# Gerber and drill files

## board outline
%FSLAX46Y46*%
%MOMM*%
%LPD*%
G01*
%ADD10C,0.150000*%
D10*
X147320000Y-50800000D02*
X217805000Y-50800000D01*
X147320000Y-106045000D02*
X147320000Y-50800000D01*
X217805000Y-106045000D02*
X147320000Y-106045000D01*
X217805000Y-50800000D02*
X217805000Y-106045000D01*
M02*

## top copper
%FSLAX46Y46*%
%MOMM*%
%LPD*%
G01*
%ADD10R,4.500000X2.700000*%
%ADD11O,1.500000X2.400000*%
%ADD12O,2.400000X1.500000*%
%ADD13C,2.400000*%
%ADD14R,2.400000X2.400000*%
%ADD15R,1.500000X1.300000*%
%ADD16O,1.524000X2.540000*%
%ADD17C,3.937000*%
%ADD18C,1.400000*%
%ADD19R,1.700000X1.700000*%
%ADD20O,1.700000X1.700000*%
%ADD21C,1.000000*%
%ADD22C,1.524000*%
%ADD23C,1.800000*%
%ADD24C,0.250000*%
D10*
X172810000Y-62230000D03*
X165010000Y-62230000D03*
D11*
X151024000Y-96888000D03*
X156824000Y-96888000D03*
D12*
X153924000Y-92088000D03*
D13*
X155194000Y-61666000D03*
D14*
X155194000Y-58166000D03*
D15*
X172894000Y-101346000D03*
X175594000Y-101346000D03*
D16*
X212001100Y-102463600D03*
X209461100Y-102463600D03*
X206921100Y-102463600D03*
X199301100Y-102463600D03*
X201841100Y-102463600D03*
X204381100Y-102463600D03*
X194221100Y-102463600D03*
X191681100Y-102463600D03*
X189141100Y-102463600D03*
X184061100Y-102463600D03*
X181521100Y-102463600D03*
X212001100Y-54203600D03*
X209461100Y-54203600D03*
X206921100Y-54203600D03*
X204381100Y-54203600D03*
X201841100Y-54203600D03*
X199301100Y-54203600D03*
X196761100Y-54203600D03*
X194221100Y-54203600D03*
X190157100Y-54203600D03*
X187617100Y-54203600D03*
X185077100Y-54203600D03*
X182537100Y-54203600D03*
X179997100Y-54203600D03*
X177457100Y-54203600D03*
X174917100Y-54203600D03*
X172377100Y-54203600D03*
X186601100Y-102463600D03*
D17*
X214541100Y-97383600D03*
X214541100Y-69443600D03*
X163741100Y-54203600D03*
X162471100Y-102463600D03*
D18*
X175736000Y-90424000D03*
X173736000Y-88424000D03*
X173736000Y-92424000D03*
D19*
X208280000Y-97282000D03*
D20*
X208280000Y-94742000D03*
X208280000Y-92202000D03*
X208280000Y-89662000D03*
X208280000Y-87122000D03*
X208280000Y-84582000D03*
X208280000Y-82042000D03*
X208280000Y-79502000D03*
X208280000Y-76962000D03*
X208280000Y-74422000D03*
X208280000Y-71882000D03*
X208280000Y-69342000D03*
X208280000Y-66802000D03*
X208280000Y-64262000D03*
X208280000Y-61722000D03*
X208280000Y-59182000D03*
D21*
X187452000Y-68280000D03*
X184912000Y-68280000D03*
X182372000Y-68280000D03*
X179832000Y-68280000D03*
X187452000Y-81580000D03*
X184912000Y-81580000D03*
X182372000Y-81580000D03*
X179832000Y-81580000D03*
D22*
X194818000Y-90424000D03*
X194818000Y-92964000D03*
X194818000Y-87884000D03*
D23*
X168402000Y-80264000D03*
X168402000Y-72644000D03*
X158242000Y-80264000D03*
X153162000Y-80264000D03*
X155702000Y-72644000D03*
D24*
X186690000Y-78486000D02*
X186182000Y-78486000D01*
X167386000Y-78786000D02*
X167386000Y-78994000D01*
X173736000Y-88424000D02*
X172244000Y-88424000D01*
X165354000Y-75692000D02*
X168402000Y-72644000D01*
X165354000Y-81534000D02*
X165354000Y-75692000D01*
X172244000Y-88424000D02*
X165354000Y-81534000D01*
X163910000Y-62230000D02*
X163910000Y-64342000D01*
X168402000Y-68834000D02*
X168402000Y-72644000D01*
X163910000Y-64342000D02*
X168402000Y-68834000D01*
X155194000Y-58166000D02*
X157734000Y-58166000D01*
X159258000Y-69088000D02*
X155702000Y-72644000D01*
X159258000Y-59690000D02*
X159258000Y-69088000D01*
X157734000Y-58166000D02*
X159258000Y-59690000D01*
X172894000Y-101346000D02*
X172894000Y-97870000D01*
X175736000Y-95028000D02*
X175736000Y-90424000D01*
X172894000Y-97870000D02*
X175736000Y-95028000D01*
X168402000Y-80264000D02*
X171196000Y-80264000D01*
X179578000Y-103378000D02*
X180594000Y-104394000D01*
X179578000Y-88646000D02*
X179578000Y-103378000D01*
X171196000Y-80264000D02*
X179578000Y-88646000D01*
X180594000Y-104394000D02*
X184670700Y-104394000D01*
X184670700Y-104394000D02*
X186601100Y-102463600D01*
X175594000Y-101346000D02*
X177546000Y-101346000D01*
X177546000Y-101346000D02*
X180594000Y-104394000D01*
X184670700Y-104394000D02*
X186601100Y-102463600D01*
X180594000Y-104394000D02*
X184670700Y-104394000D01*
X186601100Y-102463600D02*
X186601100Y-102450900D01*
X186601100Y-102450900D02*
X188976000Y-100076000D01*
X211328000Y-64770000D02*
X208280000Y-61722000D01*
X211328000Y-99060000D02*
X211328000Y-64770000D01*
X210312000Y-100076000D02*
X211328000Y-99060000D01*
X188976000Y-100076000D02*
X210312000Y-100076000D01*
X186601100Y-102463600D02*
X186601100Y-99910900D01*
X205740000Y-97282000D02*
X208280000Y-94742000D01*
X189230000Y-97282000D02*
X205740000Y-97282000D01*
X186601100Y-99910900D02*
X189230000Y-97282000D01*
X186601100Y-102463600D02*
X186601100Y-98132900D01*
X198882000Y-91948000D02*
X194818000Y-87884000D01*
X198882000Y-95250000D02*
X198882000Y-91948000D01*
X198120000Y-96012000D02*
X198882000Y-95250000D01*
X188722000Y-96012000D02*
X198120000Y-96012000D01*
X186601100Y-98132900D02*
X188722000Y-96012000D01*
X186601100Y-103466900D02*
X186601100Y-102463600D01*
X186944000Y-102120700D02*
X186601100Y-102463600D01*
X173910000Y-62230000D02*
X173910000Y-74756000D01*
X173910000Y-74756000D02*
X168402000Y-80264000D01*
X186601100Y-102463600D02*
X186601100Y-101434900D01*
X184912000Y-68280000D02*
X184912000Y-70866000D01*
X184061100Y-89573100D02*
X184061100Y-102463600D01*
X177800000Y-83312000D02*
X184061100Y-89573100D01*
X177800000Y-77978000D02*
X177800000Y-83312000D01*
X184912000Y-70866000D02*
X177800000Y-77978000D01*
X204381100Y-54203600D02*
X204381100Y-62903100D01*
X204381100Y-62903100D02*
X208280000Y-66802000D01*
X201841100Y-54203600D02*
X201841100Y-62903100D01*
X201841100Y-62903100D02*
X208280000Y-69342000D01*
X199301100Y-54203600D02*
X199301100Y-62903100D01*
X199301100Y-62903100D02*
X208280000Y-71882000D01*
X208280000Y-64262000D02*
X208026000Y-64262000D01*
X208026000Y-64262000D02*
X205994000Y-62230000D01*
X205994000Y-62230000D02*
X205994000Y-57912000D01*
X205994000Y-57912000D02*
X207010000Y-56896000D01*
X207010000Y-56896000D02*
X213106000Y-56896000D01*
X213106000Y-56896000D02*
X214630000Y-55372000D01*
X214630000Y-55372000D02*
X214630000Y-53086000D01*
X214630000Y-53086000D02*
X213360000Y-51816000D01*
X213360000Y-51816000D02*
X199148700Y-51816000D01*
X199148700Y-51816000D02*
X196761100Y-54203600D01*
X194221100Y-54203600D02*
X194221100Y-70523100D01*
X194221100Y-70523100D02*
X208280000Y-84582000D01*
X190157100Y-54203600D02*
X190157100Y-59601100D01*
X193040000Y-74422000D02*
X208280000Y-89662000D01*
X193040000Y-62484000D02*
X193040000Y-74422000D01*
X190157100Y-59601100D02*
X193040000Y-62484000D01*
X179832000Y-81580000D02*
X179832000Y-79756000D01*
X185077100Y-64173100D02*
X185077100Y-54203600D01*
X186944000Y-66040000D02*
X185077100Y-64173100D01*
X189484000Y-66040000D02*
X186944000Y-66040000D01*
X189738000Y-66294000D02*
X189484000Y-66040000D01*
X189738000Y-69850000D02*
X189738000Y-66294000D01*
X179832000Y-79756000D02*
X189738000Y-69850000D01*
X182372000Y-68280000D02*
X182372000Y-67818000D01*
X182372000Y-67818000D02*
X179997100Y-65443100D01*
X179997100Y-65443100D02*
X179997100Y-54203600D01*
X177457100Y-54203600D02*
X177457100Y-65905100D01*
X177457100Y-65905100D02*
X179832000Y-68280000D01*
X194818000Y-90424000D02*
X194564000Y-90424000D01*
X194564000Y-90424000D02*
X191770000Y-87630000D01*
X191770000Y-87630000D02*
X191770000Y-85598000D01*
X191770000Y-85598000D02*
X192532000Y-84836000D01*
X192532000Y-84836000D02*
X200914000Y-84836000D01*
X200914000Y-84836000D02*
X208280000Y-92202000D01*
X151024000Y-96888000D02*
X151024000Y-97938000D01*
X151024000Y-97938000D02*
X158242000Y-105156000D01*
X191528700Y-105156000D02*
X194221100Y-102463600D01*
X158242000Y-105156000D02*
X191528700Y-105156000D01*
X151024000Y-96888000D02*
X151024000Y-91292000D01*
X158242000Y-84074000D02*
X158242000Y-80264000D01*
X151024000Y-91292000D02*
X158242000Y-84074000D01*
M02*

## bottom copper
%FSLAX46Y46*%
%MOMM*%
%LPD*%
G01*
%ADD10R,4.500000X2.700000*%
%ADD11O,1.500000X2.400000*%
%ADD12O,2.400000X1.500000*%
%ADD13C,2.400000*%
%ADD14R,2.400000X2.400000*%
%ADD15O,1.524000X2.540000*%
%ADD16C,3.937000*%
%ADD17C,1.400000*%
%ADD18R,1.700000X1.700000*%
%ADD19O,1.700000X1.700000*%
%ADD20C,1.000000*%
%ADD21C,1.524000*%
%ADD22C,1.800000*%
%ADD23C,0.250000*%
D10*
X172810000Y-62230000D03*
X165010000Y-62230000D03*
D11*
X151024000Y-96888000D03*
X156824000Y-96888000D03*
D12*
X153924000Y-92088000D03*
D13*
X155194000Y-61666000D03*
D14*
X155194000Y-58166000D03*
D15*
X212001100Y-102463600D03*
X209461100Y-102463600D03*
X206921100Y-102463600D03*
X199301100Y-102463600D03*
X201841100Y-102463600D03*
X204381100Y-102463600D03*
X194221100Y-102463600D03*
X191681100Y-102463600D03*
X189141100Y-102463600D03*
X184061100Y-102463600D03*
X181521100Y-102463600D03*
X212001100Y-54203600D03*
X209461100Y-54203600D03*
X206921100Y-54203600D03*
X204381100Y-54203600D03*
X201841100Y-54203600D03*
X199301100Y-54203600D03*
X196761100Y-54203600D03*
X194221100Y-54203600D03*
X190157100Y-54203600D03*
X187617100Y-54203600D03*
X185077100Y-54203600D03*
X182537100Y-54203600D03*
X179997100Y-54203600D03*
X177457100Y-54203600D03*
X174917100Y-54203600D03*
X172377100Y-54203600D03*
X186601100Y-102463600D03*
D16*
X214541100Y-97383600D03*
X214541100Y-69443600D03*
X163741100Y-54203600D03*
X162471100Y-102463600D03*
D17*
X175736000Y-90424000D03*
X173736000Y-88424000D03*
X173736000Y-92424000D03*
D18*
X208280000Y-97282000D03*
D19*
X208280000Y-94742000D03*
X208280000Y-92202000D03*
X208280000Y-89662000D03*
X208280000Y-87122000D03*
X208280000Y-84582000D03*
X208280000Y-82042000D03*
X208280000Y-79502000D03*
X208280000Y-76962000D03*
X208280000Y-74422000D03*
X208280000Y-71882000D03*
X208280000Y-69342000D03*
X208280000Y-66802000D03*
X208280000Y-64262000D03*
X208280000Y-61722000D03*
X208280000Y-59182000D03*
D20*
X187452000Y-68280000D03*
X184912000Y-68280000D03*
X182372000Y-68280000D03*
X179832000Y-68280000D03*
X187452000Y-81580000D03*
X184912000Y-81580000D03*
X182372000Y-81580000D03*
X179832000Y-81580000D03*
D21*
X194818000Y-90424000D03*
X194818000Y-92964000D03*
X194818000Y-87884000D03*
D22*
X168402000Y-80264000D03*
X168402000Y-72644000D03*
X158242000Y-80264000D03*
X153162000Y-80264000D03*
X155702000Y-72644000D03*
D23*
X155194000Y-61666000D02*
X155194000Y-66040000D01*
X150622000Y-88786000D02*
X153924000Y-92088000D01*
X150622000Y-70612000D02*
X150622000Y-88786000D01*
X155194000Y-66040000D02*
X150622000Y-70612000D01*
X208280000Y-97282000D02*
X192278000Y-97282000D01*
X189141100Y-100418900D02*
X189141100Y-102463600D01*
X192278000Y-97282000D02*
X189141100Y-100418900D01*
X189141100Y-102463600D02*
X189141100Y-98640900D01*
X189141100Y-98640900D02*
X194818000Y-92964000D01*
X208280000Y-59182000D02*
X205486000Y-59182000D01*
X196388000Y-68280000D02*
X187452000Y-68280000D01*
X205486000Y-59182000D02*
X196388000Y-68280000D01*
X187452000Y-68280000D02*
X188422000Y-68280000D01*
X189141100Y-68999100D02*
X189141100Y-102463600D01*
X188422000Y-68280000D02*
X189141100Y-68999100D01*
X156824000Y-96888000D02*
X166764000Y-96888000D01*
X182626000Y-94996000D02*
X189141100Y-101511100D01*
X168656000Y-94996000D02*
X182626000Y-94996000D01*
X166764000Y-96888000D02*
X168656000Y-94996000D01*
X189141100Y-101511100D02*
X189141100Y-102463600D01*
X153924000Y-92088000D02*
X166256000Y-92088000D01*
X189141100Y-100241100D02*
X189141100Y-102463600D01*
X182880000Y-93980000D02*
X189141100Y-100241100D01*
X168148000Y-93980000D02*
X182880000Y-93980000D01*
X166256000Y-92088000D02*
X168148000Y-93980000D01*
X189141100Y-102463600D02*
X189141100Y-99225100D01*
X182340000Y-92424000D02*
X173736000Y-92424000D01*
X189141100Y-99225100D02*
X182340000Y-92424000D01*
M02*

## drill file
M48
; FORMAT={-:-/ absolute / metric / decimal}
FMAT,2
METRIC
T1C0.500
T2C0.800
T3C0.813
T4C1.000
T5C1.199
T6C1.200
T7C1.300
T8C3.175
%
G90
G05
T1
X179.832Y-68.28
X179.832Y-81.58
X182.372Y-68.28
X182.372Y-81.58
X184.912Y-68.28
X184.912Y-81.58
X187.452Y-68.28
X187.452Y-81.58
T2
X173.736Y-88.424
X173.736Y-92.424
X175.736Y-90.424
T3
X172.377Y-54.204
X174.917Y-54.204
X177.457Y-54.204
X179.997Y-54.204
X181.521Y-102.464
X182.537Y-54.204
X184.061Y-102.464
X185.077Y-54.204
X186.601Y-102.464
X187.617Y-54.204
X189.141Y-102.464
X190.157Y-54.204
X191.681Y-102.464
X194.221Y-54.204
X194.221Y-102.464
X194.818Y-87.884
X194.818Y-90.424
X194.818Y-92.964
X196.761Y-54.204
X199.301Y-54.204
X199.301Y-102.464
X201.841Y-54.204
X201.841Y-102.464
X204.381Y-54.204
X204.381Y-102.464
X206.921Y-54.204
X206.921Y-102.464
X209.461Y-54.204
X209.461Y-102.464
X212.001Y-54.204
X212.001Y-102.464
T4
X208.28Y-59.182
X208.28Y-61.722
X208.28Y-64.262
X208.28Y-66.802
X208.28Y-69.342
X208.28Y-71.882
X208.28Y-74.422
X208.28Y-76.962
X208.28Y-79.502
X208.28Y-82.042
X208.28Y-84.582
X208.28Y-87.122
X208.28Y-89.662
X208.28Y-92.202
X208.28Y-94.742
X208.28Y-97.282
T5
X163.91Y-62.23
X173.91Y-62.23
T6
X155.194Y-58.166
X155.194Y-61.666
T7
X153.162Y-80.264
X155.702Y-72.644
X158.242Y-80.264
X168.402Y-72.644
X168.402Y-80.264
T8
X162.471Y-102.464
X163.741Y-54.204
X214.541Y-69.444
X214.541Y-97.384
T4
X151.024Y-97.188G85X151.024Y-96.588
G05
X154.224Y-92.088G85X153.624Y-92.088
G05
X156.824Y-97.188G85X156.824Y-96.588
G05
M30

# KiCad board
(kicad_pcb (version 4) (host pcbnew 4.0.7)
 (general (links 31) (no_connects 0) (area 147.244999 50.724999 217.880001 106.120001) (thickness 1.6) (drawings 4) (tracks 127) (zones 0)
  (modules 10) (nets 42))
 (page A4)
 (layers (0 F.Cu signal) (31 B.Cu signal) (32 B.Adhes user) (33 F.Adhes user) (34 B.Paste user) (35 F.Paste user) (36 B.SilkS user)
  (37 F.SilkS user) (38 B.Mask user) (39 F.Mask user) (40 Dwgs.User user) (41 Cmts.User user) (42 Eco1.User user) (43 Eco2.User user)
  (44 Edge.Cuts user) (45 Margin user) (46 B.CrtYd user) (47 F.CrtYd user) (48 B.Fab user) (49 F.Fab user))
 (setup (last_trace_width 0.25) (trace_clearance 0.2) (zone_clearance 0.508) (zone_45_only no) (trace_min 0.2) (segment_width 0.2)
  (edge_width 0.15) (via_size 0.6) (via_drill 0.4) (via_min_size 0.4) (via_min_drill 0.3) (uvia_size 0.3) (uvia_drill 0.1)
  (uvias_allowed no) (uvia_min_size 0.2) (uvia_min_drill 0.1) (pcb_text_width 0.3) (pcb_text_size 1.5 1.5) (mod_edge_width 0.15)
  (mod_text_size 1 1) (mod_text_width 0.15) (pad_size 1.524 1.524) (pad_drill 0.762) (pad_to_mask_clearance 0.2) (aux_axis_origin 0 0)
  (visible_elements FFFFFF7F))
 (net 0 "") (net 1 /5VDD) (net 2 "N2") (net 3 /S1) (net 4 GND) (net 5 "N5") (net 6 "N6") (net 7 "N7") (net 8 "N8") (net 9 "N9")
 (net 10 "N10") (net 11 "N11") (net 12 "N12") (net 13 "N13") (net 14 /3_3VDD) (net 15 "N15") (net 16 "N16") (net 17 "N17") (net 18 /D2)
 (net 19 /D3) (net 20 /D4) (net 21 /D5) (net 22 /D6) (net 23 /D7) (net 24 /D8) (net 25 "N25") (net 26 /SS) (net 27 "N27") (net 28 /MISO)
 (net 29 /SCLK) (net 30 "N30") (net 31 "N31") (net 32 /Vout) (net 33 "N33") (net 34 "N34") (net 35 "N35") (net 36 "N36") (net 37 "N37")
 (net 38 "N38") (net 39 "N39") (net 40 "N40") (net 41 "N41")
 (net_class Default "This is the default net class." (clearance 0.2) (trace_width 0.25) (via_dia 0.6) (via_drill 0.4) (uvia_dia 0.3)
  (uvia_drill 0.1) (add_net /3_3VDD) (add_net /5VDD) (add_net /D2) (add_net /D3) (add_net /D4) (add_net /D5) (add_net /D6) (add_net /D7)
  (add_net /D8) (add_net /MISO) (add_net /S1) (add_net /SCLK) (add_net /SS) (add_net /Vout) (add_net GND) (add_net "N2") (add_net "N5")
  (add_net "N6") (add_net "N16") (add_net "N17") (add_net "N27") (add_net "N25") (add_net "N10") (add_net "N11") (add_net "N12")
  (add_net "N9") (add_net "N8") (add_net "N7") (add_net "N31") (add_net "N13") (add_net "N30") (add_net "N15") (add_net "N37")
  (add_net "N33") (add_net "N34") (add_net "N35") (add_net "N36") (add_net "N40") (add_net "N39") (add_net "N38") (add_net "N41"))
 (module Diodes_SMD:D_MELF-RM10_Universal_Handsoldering (layer F.Cu) (at 168.91 62.23 180)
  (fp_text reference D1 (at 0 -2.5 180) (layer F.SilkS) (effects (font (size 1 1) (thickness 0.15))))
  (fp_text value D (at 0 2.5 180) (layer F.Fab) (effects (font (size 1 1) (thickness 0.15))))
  (pad 1 thru_hole rect (at -5 0 180) (size 4.5 2.7) (drill 1.19888 (offset 1.1 0)) (layers *.Cu *.Mask) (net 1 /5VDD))
  (pad 2 thru_hole rect (at 5 0) (size 4.5 2.7) (drill 1.19888 (offset 1.1 0)) (layers *.Cu *.Mask) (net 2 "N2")))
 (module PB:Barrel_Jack (layer F.Cu) (at 153.924 94.488 180)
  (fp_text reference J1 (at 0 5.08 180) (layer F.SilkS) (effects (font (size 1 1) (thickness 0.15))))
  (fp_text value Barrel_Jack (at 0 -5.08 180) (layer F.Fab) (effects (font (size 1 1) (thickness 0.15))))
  (pad 1 thru_hole oval (at 2.9 -2.4 180) (size 1.5 2.4) (drill oval 1 1.6) (layers *.Cu *.Mask) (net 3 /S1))
  (pad 2 thru_hole oval (at -2.9 -2.4 180) (size 1.5 2.4) (drill oval 1 1.6) (layers *.Cu *.Mask) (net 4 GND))
  (pad 3 thru_hole oval (at 0 2.4 180) (size 2.4 1.5) (drill oval 1.6 1) (layers *.Cu *.Mask) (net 4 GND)))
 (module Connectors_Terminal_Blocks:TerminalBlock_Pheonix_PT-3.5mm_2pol (layer F.Cu) (at 155.194 58.166 270)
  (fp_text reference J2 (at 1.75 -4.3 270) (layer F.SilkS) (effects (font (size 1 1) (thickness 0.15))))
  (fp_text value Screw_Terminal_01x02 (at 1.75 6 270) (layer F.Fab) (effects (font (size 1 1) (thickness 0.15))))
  (pad 2 thru_hole circle (at 3.5 0 270) (size 2.4 2.4) (drill 1.2) (layers *.Cu *.Mask) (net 4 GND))
  (pad 1 thru_hole rect (at 0 0 270) (size 2.4 2.4) (drill 1.2) (layers *.Cu *.Mask) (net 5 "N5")))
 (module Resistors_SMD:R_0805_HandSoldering (layer F.Cu) (at 174.244 101.346)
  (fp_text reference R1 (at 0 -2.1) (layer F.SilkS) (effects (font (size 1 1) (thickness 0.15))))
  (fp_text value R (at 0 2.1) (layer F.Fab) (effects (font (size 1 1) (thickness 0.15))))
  (pad 1 smd rect (at -1.35 0) (size 1.5 1.3) (layers F.Cu F.Paste F.Mask) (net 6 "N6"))
  (pad 2 smd rect (at 1.35 0) (size 1.5 1.3) (layers F.Cu F.Paste F.Mask) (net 1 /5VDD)))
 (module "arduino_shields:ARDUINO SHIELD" (layer F.Cu) (at 148.5011 105.0036)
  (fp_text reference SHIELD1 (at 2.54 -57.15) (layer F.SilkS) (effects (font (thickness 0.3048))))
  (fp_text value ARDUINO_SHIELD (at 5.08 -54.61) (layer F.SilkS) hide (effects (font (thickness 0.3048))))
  (pad AD5 thru_hole oval (at 63.5 -2.54 90) (size 2.54 1.524) (drill 0.8128) (layers *.Cu *.Mask F.SilkS) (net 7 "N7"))
  (pad AD4 thru_hole oval (at 60.96 -2.54 90) (size 2.54 1.524) (drill 0.8128) (layers *.Cu *.Mask F.SilkS) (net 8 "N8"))
  (pad AD3 thru_hole oval (at 58.42 -2.54 90) (size 2.54 1.524) (drill 0.8128) (layers *.Cu *.Mask F.SilkS) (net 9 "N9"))
  (pad AD0 thru_hole oval (at 50.8 -2.54 90) (size 2.54 1.524) (drill 0.8128) (layers *.Cu *.Mask F.SilkS) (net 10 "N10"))
  (pad AD1 thru_hole oval (at 53.34 -2.54 90) (size 2.54 1.524) (drill 0.8128) (layers *.Cu *.Mask F.SilkS) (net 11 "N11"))
  (pad AD2 thru_hole oval (at 55.88 -2.54 90) (size 2.54 1.524) (drill 0.8128) (layers *.Cu *.Mask F.SilkS) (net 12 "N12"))
  (pad V_IN thru_hole oval (at 45.72 -2.54 90) (size 2.54 1.524) (drill 0.8128) (layers *.Cu *.Mask F.SilkS) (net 3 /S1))
  (pad GND2 thru_hole oval (at 43.18 -2.54 90) (size 2.54 1.524) (drill 0.8128) (layers *.Cu *.Mask F.SilkS) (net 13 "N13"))
  (pad GND1 thru_hole oval (at 40.64 -2.54 90) (size 2.54 1.524) (drill 0.8128) (layers *.Cu *.Mask F.SilkS) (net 4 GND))
  (pad 3V3 thru_hole oval (at 35.56 -2.54 90) (size 2.54 1.524) (drill 0.8128) (layers *.Cu *.Mask F.SilkS) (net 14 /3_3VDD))
  (pad RST thru_hole oval (at 33.02 -2.54 90) (size 2.54 1.524) (drill 0.8128) (layers *.Cu *.Mask F.SilkS) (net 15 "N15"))
  (pad 0 thru_hole oval (at 63.5 -50.8 90) (size 2.54 1.524) (drill 0.8128) (layers *.Cu *.Mask F.SilkS) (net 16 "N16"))
  (pad 1 thru_hole oval (at 60.96 -50.8 90) (size 2.54 1.524) (drill 0.8128) (layers *.Cu *.Mask F.SilkS) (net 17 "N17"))
  (pad 2 thru_hole oval (at 58.42 -50.8 90) (size 2.54 1.524) (drill 0.8128) (layers *.Cu *.Mask F.SilkS) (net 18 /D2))
  (pad 3 thru_hole oval (at 55.88 -50.8 90) (size 2.54 1.524) (drill 0.8128) (layers *.Cu *.Mask F.SilkS) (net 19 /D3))
  (pad 4 thru_hole oval (at 53.34 -50.8 90) (size 2.54 1.524) (drill 0.8128) (layers *.Cu *.Mask F.SilkS) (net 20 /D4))
  (pad 5 thru_hole oval (at 50.8 -50.8 90) (size 2.54 1.524) (drill 0.8128) (layers *.Cu *.Mask F.SilkS) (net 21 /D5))
  (pad 6 thru_hole oval (at 48.26 -50.8 90) (size 2.54 1.524) (drill 0.8128) (layers *.Cu *.Mask F.SilkS) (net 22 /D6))
  (pad 7 thru_hole oval (at 45.72 -50.8 90) (size 2.54 1.524) (drill 0.8128) (layers *.Cu *.Mask F.SilkS) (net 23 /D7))
  (pad 8 thru_hole oval (at 41.656 -50.8 90) (size 2.54 1.524) (drill 0.8128) (layers *.Cu *.Mask F.SilkS) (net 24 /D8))
  (pad 9 thru_hole oval (at 39.116 -50.8 90) (size 2.54 1.524) (drill 0.8128) (layers *.Cu *.Mask F.SilkS) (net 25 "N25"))
  (pad 10 thru_hole oval (at 36.576 -50.8 90) (size 2.54 1.524) (drill 0.8128) (layers *.Cu *.Mask F.SilkS) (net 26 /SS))
  (pad 11 thru_hole oval (at 34.036 -50.8 90) (size 2.54 1.524) (drill 0.8128) (layers *.Cu *.Mask F.SilkS) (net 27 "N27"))
  (pad 12 thru_hole oval (at 31.496 -50.8 90) (size 2.54 1.524) (drill 0.8128) (layers *.Cu *.Mask F.SilkS) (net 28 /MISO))
  (pad 13 thru_hole oval (at 28.956 -50.8 90) (size 2.54 1.524) (drill 0.8128) (layers *.Cu *.Mask F.SilkS) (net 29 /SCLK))
  (pad GND3 thru_hole oval (at 26.416 -50.8 90) (size 2.54 1.524) (drill 0.8128) (layers *.Cu *.Mask F.SilkS) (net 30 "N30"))
  (pad AREF thru_hole oval (at 23.876 -50.8 90) (size 2.54 1.524) (drill 0.8128) (layers *.Cu *.Mask F.SilkS) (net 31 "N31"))
  (pad 5V thru_hole oval (at 38.1 -2.54 90) (size 2.54 1.524) (drill 0.8128) (layers *.Cu *.Mask F.SilkS) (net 1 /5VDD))
  (pad "" thru_hole circle (at 66.04 -7.62 90) (size 3.937 3.937) (drill 3.175) (layers *.Cu *.Mask F.SilkS))
  (pad "" thru_hole circle (at 66.04 -35.56 90) (size 3.937 3.937) (drill 3.175) (layers *.Cu *.Mask F.SilkS))
  (pad "" thru_hole circle (at 15.24 -50.8 90) (size 3.937 3.937) (drill 3.175) (layers *.Cu *.Mask F.SilkS))
  (pad "" thru_hole circle (at 13.97 -2.54 90) (size 3.937 3.937) (drill 3.175) (layers *.Cu *.Mask F.SilkS)))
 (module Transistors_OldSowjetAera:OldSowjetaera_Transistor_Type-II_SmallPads (layer F.Cu) (at 173.736 90.424 270)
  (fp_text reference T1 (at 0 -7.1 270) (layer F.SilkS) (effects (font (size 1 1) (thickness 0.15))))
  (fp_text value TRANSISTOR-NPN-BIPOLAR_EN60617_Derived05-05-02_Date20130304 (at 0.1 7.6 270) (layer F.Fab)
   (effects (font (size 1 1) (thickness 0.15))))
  (pad 2 thru_hole circle (at 0 -2 270) (size 1.4 1.4) (drill 0.8) (layers *.Cu *.Mask) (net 6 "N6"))
  (pad 1 thru_hole circle (at -2 0 270) (size 1.4 1.4) (drill 0.8) (layers *.Cu *.Mask) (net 2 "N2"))
  (pad 3 thru_hole circle (at 2 0 270) (size 1.4 1.4) (drill 0.8) (layers *.Cu *.Mask) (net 4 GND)))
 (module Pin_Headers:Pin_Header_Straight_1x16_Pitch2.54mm (layer F.Cu) (at 208.28 97.282 180)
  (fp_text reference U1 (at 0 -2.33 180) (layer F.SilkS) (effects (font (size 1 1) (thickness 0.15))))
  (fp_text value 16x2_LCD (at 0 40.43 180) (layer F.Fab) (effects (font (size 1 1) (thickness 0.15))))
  (pad 1 thru_hole rect (at 0 0 180) (size 1.7 1.7) (drill 1) (layers *.Cu *.Mask) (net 4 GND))
  (pad 2 thru_hole oval (at 0 2.54 180) (size 1.7 1.7) (drill 1) (layers *.Cu *.Mask) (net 1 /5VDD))
  (pad 3 thru_hole oval (at 0 5.08 180) (size 1.7 1.7) (drill 1) (layers *.Cu *.Mask) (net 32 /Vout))
  (pad 4 thru_hole oval (at 0 7.62 180) (size 1.7 1.7) (drill 1) (layers *.Cu *.Mask) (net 24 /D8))
  (pad 5 thru_hole oval (at 0 10.16 180) (size 1.7 1.7) (drill 1) (layers *.Cu *.Mask) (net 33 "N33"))
  (pad 6 thru_hole oval (at 0 12.7 180) (size 1.7 1.7) (drill 1) (layers *.Cu *.Mask) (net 23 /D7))
  (pad 7 thru_hole oval (at 0 15.24 180) (size 1.7 1.7) (drill 1) (layers *.Cu *.Mask) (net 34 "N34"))
  (pad 8 thru_hole oval (at 0 17.78 180) (size 1.7 1.7) (drill 1) (layers *.Cu *.Mask) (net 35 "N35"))
  (pad 9 thru_hole oval (at 0 20.32 180) (size 1.7 1.7) (drill 1) (layers *.Cu *.Mask) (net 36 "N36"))
  (pad 10 thru_hole oval (at 0 22.86 180) (size 1.7 1.7) (drill 1) (layers *.Cu *.Mask) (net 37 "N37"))
  (pad 11 thru_hole oval (at 0 25.4 180) (size 1.7 1.7) (drill 1) (layers *.Cu *.Mask) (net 21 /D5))
  (pad 12 thru_hole oval (at 0 27.94 180) (size 1.7 1.7) (drill 1) (layers *.Cu *.Mask) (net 20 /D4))
  (pad 13 thru_hole oval (at 0 30.48 180) (size 1.7 1.7) (drill 1) (layers *.Cu *.Mask) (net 19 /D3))
  (pad 14 thru_hole oval (at 0 33.02 180) (size 1.7 1.7) (drill 1) (layers *.Cu *.Mask) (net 22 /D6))
  (pad 15 thru_hole oval (at 0 35.56 180) (size 1.7 1.7) (drill 1) (layers *.Cu *.Mask) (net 1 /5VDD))
  (pad 16 thru_hole oval (at 0 38.1 180) (size 1.7 1.7) (drill 1) (layers *.Cu *.Mask) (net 4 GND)))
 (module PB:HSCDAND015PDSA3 (layer F.Cu) (at 183.642 74.93 270)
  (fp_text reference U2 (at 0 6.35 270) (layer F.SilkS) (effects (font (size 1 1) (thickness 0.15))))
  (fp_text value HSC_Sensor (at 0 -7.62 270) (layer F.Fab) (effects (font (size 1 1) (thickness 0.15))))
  (pad 1 thru_hole circle (at -6.65 -3.81 270) (size 1 1) (drill 0.5) (layers *.Cu *.Mask) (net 4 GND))
  (pad 2 thru_hole circle (at -6.65 -1.27 270) (size 1 1) (drill 0.5) (layers *.Cu *.Mask) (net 14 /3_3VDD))
  (pad 3 thru_hole circle (at -6.65 1.27 270) (size 1 1) (drill 0.5) (layers *.Cu *.Mask) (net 28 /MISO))
  (pad 4 thru_hole circle (at -6.65 3.81 270) (size 1 1) (drill 0.5) (layers *.Cu *.Mask) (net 29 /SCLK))
  (pad 8 thru_hole circle (at 6.65 -3.81 270) (size 1 1) (drill 0.5) (layers *.Cu *.Mask) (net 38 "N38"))
  (pad 7 thru_hole circle (at 6.65 -1.27 270) (size 1 1) (drill 0.5) (layers *.Cu *.Mask) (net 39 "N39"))
  (pad 6 thru_hole circle (at 6.65 1.27 270) (size 1 1) (drill 0.5) (layers *.Cu *.Mask) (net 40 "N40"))
  (pad 5 thru_hole circle (at 6.65 3.81 270) (size 1 1) (drill 0.5) (layers *.Cu *.Mask) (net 26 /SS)))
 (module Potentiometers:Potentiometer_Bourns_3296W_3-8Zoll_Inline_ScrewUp (layer F.Cu) (at 194.818 87.884 180)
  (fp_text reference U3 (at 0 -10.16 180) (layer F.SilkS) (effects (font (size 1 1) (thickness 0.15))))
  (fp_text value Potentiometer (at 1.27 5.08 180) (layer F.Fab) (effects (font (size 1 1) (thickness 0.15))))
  (pad 2 thru_hole circle (at 0 -2.54 180) (size 1.524 1.524) (drill 0.8128) (layers *.Cu *.Mask) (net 32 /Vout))
  (pad 3 thru_hole circle (at 0 -5.08 180) (size 1.524 1.524) (drill 0.8128) (layers *.Cu *.Mask) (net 4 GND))
  (pad 1 thru_hole circle (at 0 0 180) (size 1.524 1.524) (drill 0.8128) (layers *.Cu *.Mask) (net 1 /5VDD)))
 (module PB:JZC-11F (layer F.Cu) (at 162.052 76.454 90)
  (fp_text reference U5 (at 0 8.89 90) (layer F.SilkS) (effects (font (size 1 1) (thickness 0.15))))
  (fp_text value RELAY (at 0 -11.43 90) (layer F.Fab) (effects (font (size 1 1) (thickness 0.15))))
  (pad 1 thru_hole circle (at -3.81 6.35 90) (size 1.8 1.8) (drill 1.3) (layers *.Cu *.Mask) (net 1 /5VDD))
  (pad 2 thru_hole circle (at 3.81 6.35 90) (size 1.8 1.8) (drill 1.3) (layers *.Cu *.Mask) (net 2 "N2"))
  (pad 3 thru_hole circle (at -3.81 -3.81 90) (size 1.8 1.8) (drill 1.3) (layers *.Cu *.Mask) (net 3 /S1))
  (pad 4 thru_hole circle (at -3.81 -8.89 90) (size 1.8 1.8) (drill 1.3) (layers *.Cu *.Mask) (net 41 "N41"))
  (pad 5 thru_hole circle (at 3.81 -6.35 90) (size 1.8 1.8) (drill 1.3) (layers *.Cu *.Mask) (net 5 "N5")))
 (gr_line (start 147.32 50.8) (end 217.805 50.8) (angle 90) (layer Edge.Cuts) (width 0.15))
 (gr_line (start 147.32 106.045) (end 147.32 50.8) (angle 90) (layer Edge.Cuts) (width 0.15))
 (gr_line (start 217.805 106.045) (end 147.32 106.045) (angle 90) (layer Edge.Cuts) (width 0.15))
 (gr_line (start 217.805 50.8) (end 217.805 106.045) (angle 90) (layer Edge.Cuts) (width 0.15))
 (segment (start 186.69 78.486) (end 186.182 78.486) (width 0.25) (layer F.Cu) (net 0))
 (segment (start 167.386 78.786) (end 167.386 78.994) (width 0.25) (layer F.Cu) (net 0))
 (segment (start 173.736 88.424) (end 172.244 88.424) (width 0.25) (layer F.Cu) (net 2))
 (segment (start 165.354 75.692) (end 168.402 72.644) (width 0.25) (layer F.Cu) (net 2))
 (segment (start 165.354 81.534) (end 165.354 75.692) (width 0.25) (layer F.Cu) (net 2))
 (segment (start 172.244 88.424) (end 165.354 81.534) (width 0.25) (layer F.Cu) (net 2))
 (segment (start 163.91 62.23) (end 163.91 64.342) (width 0.25) (layer F.Cu) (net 2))
 (segment (start 168.402 68.834) (end 168.402 72.644) (width 0.25) (layer F.Cu) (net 2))
 (segment (start 163.91 64.342) (end 168.402 68.834) (width 0.25) (layer F.Cu) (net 2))
 (segment (start 155.194 58.166) (end 157.734 58.166) (width 0.25) (layer F.Cu) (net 5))
 (segment (start 159.258 69.088) (end 155.702 72.644) (width 0.25) (layer F.Cu) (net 5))
 (segment (start 159.258 59.69) (end 159.258 69.088) (width 0.25) (layer F.Cu) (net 5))
 (segment (start 157.734 58.166) (end 159.258 59.69) (width 0.25) (layer F.Cu) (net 5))
 (segment (start 155.194 61.666) (end 155.194 66.04) (width 0.25) (layer B.Cu) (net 4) (status 400000))
 (segment (start 150.622 88.786) (end 153.924 92.088) (width 0.25) (layer B.Cu) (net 4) (status 800000))
 (segment (start 150.622 70.612) (end 150.622 88.786) (width 0.25) (layer B.Cu) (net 4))
 (segment (start 155.194 66.04) (end 150.622 70.612) (width 0.25) (layer B.Cu) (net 4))
 (segment (start 208.28 97.282) (end 192.278 97.282) (width 0.25) (layer B.Cu) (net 4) (status 400000))
 (segment (start 189.1411 100.4189) (end 189.1411 102.4636) (width 0.25) (layer B.Cu) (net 4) (status 800000))
 (segment (start 192.278 97.282) (end 189.1411 100.4189) (width 0.25) (layer B.Cu) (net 4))
 (segment (start 189.1411 102.4636) (end 189.1411 98.6409) (width 0.25) (layer B.Cu) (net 4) (status 400000))
 (segment (start 189.1411 98.6409) (end 194.818 92.964) (width 0.25) (layer B.Cu) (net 4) (status 800000))
 (segment (start 208.28 59.182) (end 205.486 59.182) (width 0.25) (layer B.Cu) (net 4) (status 400000))
 (segment (start 196.388 68.28) (end 187.452 68.28) (width 0.25) (layer B.Cu) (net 4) (status 800000))
 (segment (start 205.486 59.182) (end 196.388 68.28) (width 0.25) (layer B.Cu) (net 4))
 (segment (start 187.452 68.28) (end 188.422 68.28) (width 0.25) (layer B.Cu) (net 4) (status 400000))
 (segment (start 189.1411 68.9991) (end 189.1411 102.4636) (width 0.25) (layer B.Cu) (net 4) (status 800000))
 (segment (start 188.422 68.28) (end 189.1411 68.9991) (width 0.25) (layer B.Cu) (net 4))
 (segment (start 156.824 96.888) (end 166.764 96.888) (width 0.25) (layer B.Cu) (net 4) (status 400000))
 (segment (start 182.626 94.996) (end 189.1411 101.5111) (width 0.25) (layer B.Cu) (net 4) (status 800000))
 (segment (start 168.656 94.996) (end 182.626 94.996) (width 0.25) (layer B.Cu) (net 4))
 (segment (start 166.764 96.888) (end 168.656 94.996) (width 0.25) (layer B.Cu) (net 4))
 (segment (start 189.1411 101.5111) (end 189.1411 102.4636) (width 0.25) (layer B.Cu) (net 4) (status C00000))
 (segment (start 153.924 92.088) (end 166.256 92.088) (width 0.25) (layer B.Cu) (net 4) (status 400000))
 (segment (start 189.1411 100.2411) (end 189.1411 102.4636) (width 0.25) (layer B.Cu) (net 4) (status 800000))
 (segment (start 182.88 93.98) (end 189.1411 100.2411) (width 0.25) (layer B.Cu) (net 4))
 (segment (start 168.148 93.98) (end 182.88 93.98) (width 0.25) (layer B.Cu) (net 4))
 (segment (start 166.256 92.088) (end 168.148 93.98) (width 0.25) (layer B.Cu) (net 4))
 (segment (start 189.1411 102.4636) (end 189.1411 99.2251) (width 0.25) (layer B.Cu) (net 4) (status 400000))
 (segment (start 182.34 92.424) (end 173.736 92.424) (width 0.25) (layer B.Cu) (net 4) (status 800000))
 (segment (start 189.1411 99.2251) (end 182.34 92.424) (width 0.25) (layer B.Cu) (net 4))
 (segment (start 172.894 101.346) (end 172.894 97.87) (width 0.25) (layer F.Cu) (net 6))
 (segment (start 175.736 95.028) (end 175.736 90.424) (width 0.25) (layer F.Cu) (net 6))
 (segment (start 172.894 97.87) (end 175.736 95.028) (width 0.25) (layer F.Cu) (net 6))
 (segment (start 168.402 80.264) (end 171.196 80.264) (width 0.25) (layer F.Cu) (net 1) (status 400000))
 (segment (start 179.578 103.378) (end 180.594 104.394) (width 0.25) (layer F.Cu) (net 1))
 (segment (start 179.578 88.646) (end 179.578 103.378) (width 0.25) (layer F.Cu) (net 1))
 (segment (start 171.196 80.264) (end 179.578 88.646) (width 0.25) (layer F.Cu) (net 1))
 (segment (start 180.594 104.394) (end 184.6707 104.394) (width 0.25) (layer F.Cu) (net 1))
 (segment (start 184.6707 104.394) (end 186.6011 102.4636) (width 0.25) (layer F.Cu) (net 1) (status 800000))
 (segment (start 175.594 101.346) (end 177.546 101.346) (width 0.25) (layer F.Cu) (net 1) (status 400000))
 (segment (start 177.546 101.346) (end 180.594 104.394) (width 0.25) (layer F.Cu) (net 1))
 (segment (start 184.6707 104.394) (end 186.6011 102.4636) (width 0.25) (layer F.Cu) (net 1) (status 800000))
 (segment (start 180.594 104.394) (end 184.6707 104.394) (width 0.25) (layer F.Cu) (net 1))
 (segment (start 186.6011 102.4636) (end 186.6011 102.4509) (width 0.25) (layer F.Cu) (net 1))
 (segment (start 186.6011 102.4509) (end 188.976 100.076) (width 0.25) (layer F.Cu) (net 1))
 (segment (start 211.328 64.77) (end 208.28 61.722) (width 0.25) (layer F.Cu) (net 1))
 (segment (start 211.328 99.06) (end 211.328 64.77) (width 0.25) (layer F.Cu) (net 1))
 (segment (start 210.312 100.076) (end 211.328 99.06) (width 0.25) (layer F.Cu) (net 1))
 (segment (start 188.976 100.076) (end 210.312 100.076) (width 0.25) (layer F.Cu) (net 1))
 (segment (start 186.6011 102.4636) (end 186.6011 99.9109) (width 0.25) (layer F.Cu) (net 1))
 (segment (start 205.74 97.282) (end 208.28 94.742) (width 0.25) (layer F.Cu) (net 1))
 (segment (start 189.23 97.282) (end 205.74 97.282) (width 0.25) (layer F.Cu) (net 1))
 (segment (start 186.6011 99.9109) (end 189.23 97.282) (width 0.25) (layer F.Cu) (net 1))
 (segment (start 186.6011 102.4636) (end 186.6011 98.1329) (width 0.25) (layer F.Cu) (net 1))
 (segment (start 198.882 91.948) (end 194.818 87.884) (width 0.25) (layer F.Cu) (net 1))
 (segment (start 198.882 95.25) (end 198.882 91.948) (width 0.25) (layer F.Cu) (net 1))
 (segment (start 198.12 96.012) (end 198.882 95.25) (width 0.25) (layer F.Cu) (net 1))
 (segment (start 188.722 96.012) (end 198.12 96.012) (width 0.25) (layer F.Cu) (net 1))
 (segment (start 186.6011 98.1329) (end 188.722 96.012) (width 0.25) (layer F.Cu) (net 1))
 (segment (start 186.6011 103.4669) (end 186.6011 102.4636) (width 0.25) (layer F.Cu) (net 1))
 (segment (start 186.944 102.1207) (end 186.6011 102.4636) (width 0.25) (layer F.Cu) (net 1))
 (segment (start 173.91 62.23) (end 173.91 74.756) (width 0.25) (layer F.Cu) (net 1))
 (segment (start 173.91 74.756) (end 168.402 80.264) (width 0.25) (layer F.Cu) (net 1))
 (segment (start 186.6011 102.4636) (end 186.6011 101.4349) (width 0.25) (layer F.Cu) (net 1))
 (segment (start 184.912 68.28) (end 184.912 70.866) (width 0.25) (layer F.Cu) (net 14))
 (segment (start 184.0611 89.5731) (end 184.0611 102.4636) (width 0.25) (layer F.Cu) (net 14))
 (segment (start 177.8 83.312) (end 184.0611 89.5731) (width 0.25) (layer F.Cu) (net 14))
 (segment (start 177.8 77.978) (end 177.8 83.312) (width 0.25) (layer F.Cu) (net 14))
 (segment (start 184.912 70.866) (end 177.8 77.978) (width 0.25) (layer F.Cu) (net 14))
 (segment (start 204.3811 54.2036) (end 204.3811 62.9031) (width 0.25) (layer F.Cu) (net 19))
 (segment (start 204.3811 62.9031) (end 208.28 66.802) (width 0.25) (layer F.Cu) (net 19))
 (segment (start 201.8411 54.2036) (end 201.8411 62.9031) (width 0.25) (layer F.Cu) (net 20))
 (segment (start 201.8411 62.9031) (end 208.28 69.342) (width 0.25) (layer F.Cu) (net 20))
 (segment (start 199.3011 54.2036) (end 199.3011 62.9031) (width 0.25) (layer F.Cu) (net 21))
 (segment (start 199.3011 62.9031) (end 208.28 71.882) (width 0.25) (layer F.Cu) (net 21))
 (segment (start 208.28 64.262) (end 208.026 64.262) (width 0.25) (layer F.Cu) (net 22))
 (segment (start 208.026 64.262) (end 205.994 62.23) (width 0.25) (layer F.Cu) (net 22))
 (segment (start 205.994 62.23) (end 205.994 57.912) (width 0.25) (layer F.Cu) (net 22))
 (segment (start 205.994 57.912) (end 207.01 56.896) (width 0.25) (layer F.Cu) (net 22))
 (segment (start 207.01 56.896) (end 213.106 56.896) (width 0.25) (layer F.Cu) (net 22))
 (segment (start 213.106 56.896) (end 214.63 55.372) (width 0.25) (layer F.Cu) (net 22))
 (segment (start 214.63 55.372) (end 214.63 53.086) (width 0.25) (layer F.Cu) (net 22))
 (segment (start 214.63 53.086) (end 213.36 51.816) (width 0.25) (layer F.Cu) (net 22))
 (segment (start 213.36 51.816) (end 199.1487 51.816) (width 0.25) (layer F.Cu) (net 22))
 (segment (start 199.1487 51.816) (end 196.7611 54.2036) (width 0.25) (layer F.Cu) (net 22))
 (segment (start 194.2211 54.2036) (end 194.2211 70.5231) (width 0.25) (layer F.Cu) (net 23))
 (segment (start 194.2211 70.5231) (end 208.28 84.582) (width 0.25) (layer F.Cu) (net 23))
 (segment (start 190.1571 54.2036) (end 190.1571 59.6011) (width 0.25) (layer F.Cu) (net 24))
 (segment (start 193.04 74.422) (end 208.28 89.662) (width 0.25) (layer F.Cu) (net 24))
 (segment (start 193.04 62.484) (end 193.04 74.422) (width 0.25) (layer F.Cu) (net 24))
 (segment (start 190.1571 59.6011) (end 193.04 62.484) (width 0.25) (layer F.Cu) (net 24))
 (segment (start 179.832 81.58) (end 179.832 79.756) (width 0.25) (layer F.Cu) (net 26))
 (segment (start 185.0771 64.1731) (end 185.0771 54.2036) (width 0.25) (layer F.Cu) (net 26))
 (segment (start 186.944 66.04) (end 185.0771 64.1731) (width 0.25) (layer F.Cu) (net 26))
 (segment (start 189.484 66.04) (end 186.944 66.04) (width 0.25) (layer F.Cu) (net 26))
 (segment (start 189.738 66.294) (end 189.484 66.04) (width 0.25) (layer F.Cu) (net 26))
 (segment (start 189.738 69.85) (end 189.738 66.294) (width 0.25) (layer F.Cu) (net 26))
 (segment (start 179.832 79.756) (end 189.738 69.85) (width 0.25) (layer F.Cu) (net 26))
 (segment (start 182.372 68.28) (end 182.372 67.818) (width 0.25) (layer F.Cu) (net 28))
 (segment (start 182.372 67.818) (end 179.9971 65.4431) (width 0.25) (layer F.Cu) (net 28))
 (segment (start 179.9971 65.4431) (end 179.9971 54.2036) (width 0.25) (layer F.Cu) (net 28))
 (segment (start 177.4571 54.2036) (end 177.4571 65.9051) (width 0.25) (layer F.Cu) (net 29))
 (segment (start 177.4571 65.9051) (end 179.832 68.28) (width 0.25) (layer F.Cu) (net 29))
 (segment (start 194.818 90.424) (end 194.564 90.424) (width 0.25) (layer F.Cu) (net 32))
 (segment (start 194.564 90.424) (end 191.77 87.63) (width 0.25) (layer F.Cu) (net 32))
 (segment (start 191.77 87.63) (end 191.77 85.598) (width 0.25) (layer F.Cu) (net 32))
 (segment (start 191.77 85.598) (end 192.532 84.836) (width 0.25) (layer F.Cu) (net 32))
 (segment (start 192.532 84.836) (end 200.914 84.836) (width 0.25) (layer F.Cu) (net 32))
 (segment (start 200.914 84.836) (end 208.28 92.202) (width 0.25) (layer F.Cu) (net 32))
 (segment (start 151.024 96.888) (end 151.024 97.938) (width 0.25) (layer F.Cu) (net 3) (status C00000))
 (segment (start 151.024 97.938) (end 158.242 105.156) (width 0.25) (layer F.Cu) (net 3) (status 400000))
 (segment (start 191.5287 105.156) (end 194.2211 102.4636) (width 0.25) (layer F.Cu) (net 3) (status 800000))
 (segment (start 158.242 105.156) (end 191.5287 105.156) (width 0.25) (layer F.Cu) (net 3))
 (segment (start 151.024 96.888) (end 151.024 91.292) (width 0.25) (layer F.Cu) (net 3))
 (segment (start 158.242 84.074) (end 158.242 80.264) (width 0.25) (layer F.Cu) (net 3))
 (segment (start 151.024 91.292) (end 158.242 84.074) (width 0.25) (layer F.Cu) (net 3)))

